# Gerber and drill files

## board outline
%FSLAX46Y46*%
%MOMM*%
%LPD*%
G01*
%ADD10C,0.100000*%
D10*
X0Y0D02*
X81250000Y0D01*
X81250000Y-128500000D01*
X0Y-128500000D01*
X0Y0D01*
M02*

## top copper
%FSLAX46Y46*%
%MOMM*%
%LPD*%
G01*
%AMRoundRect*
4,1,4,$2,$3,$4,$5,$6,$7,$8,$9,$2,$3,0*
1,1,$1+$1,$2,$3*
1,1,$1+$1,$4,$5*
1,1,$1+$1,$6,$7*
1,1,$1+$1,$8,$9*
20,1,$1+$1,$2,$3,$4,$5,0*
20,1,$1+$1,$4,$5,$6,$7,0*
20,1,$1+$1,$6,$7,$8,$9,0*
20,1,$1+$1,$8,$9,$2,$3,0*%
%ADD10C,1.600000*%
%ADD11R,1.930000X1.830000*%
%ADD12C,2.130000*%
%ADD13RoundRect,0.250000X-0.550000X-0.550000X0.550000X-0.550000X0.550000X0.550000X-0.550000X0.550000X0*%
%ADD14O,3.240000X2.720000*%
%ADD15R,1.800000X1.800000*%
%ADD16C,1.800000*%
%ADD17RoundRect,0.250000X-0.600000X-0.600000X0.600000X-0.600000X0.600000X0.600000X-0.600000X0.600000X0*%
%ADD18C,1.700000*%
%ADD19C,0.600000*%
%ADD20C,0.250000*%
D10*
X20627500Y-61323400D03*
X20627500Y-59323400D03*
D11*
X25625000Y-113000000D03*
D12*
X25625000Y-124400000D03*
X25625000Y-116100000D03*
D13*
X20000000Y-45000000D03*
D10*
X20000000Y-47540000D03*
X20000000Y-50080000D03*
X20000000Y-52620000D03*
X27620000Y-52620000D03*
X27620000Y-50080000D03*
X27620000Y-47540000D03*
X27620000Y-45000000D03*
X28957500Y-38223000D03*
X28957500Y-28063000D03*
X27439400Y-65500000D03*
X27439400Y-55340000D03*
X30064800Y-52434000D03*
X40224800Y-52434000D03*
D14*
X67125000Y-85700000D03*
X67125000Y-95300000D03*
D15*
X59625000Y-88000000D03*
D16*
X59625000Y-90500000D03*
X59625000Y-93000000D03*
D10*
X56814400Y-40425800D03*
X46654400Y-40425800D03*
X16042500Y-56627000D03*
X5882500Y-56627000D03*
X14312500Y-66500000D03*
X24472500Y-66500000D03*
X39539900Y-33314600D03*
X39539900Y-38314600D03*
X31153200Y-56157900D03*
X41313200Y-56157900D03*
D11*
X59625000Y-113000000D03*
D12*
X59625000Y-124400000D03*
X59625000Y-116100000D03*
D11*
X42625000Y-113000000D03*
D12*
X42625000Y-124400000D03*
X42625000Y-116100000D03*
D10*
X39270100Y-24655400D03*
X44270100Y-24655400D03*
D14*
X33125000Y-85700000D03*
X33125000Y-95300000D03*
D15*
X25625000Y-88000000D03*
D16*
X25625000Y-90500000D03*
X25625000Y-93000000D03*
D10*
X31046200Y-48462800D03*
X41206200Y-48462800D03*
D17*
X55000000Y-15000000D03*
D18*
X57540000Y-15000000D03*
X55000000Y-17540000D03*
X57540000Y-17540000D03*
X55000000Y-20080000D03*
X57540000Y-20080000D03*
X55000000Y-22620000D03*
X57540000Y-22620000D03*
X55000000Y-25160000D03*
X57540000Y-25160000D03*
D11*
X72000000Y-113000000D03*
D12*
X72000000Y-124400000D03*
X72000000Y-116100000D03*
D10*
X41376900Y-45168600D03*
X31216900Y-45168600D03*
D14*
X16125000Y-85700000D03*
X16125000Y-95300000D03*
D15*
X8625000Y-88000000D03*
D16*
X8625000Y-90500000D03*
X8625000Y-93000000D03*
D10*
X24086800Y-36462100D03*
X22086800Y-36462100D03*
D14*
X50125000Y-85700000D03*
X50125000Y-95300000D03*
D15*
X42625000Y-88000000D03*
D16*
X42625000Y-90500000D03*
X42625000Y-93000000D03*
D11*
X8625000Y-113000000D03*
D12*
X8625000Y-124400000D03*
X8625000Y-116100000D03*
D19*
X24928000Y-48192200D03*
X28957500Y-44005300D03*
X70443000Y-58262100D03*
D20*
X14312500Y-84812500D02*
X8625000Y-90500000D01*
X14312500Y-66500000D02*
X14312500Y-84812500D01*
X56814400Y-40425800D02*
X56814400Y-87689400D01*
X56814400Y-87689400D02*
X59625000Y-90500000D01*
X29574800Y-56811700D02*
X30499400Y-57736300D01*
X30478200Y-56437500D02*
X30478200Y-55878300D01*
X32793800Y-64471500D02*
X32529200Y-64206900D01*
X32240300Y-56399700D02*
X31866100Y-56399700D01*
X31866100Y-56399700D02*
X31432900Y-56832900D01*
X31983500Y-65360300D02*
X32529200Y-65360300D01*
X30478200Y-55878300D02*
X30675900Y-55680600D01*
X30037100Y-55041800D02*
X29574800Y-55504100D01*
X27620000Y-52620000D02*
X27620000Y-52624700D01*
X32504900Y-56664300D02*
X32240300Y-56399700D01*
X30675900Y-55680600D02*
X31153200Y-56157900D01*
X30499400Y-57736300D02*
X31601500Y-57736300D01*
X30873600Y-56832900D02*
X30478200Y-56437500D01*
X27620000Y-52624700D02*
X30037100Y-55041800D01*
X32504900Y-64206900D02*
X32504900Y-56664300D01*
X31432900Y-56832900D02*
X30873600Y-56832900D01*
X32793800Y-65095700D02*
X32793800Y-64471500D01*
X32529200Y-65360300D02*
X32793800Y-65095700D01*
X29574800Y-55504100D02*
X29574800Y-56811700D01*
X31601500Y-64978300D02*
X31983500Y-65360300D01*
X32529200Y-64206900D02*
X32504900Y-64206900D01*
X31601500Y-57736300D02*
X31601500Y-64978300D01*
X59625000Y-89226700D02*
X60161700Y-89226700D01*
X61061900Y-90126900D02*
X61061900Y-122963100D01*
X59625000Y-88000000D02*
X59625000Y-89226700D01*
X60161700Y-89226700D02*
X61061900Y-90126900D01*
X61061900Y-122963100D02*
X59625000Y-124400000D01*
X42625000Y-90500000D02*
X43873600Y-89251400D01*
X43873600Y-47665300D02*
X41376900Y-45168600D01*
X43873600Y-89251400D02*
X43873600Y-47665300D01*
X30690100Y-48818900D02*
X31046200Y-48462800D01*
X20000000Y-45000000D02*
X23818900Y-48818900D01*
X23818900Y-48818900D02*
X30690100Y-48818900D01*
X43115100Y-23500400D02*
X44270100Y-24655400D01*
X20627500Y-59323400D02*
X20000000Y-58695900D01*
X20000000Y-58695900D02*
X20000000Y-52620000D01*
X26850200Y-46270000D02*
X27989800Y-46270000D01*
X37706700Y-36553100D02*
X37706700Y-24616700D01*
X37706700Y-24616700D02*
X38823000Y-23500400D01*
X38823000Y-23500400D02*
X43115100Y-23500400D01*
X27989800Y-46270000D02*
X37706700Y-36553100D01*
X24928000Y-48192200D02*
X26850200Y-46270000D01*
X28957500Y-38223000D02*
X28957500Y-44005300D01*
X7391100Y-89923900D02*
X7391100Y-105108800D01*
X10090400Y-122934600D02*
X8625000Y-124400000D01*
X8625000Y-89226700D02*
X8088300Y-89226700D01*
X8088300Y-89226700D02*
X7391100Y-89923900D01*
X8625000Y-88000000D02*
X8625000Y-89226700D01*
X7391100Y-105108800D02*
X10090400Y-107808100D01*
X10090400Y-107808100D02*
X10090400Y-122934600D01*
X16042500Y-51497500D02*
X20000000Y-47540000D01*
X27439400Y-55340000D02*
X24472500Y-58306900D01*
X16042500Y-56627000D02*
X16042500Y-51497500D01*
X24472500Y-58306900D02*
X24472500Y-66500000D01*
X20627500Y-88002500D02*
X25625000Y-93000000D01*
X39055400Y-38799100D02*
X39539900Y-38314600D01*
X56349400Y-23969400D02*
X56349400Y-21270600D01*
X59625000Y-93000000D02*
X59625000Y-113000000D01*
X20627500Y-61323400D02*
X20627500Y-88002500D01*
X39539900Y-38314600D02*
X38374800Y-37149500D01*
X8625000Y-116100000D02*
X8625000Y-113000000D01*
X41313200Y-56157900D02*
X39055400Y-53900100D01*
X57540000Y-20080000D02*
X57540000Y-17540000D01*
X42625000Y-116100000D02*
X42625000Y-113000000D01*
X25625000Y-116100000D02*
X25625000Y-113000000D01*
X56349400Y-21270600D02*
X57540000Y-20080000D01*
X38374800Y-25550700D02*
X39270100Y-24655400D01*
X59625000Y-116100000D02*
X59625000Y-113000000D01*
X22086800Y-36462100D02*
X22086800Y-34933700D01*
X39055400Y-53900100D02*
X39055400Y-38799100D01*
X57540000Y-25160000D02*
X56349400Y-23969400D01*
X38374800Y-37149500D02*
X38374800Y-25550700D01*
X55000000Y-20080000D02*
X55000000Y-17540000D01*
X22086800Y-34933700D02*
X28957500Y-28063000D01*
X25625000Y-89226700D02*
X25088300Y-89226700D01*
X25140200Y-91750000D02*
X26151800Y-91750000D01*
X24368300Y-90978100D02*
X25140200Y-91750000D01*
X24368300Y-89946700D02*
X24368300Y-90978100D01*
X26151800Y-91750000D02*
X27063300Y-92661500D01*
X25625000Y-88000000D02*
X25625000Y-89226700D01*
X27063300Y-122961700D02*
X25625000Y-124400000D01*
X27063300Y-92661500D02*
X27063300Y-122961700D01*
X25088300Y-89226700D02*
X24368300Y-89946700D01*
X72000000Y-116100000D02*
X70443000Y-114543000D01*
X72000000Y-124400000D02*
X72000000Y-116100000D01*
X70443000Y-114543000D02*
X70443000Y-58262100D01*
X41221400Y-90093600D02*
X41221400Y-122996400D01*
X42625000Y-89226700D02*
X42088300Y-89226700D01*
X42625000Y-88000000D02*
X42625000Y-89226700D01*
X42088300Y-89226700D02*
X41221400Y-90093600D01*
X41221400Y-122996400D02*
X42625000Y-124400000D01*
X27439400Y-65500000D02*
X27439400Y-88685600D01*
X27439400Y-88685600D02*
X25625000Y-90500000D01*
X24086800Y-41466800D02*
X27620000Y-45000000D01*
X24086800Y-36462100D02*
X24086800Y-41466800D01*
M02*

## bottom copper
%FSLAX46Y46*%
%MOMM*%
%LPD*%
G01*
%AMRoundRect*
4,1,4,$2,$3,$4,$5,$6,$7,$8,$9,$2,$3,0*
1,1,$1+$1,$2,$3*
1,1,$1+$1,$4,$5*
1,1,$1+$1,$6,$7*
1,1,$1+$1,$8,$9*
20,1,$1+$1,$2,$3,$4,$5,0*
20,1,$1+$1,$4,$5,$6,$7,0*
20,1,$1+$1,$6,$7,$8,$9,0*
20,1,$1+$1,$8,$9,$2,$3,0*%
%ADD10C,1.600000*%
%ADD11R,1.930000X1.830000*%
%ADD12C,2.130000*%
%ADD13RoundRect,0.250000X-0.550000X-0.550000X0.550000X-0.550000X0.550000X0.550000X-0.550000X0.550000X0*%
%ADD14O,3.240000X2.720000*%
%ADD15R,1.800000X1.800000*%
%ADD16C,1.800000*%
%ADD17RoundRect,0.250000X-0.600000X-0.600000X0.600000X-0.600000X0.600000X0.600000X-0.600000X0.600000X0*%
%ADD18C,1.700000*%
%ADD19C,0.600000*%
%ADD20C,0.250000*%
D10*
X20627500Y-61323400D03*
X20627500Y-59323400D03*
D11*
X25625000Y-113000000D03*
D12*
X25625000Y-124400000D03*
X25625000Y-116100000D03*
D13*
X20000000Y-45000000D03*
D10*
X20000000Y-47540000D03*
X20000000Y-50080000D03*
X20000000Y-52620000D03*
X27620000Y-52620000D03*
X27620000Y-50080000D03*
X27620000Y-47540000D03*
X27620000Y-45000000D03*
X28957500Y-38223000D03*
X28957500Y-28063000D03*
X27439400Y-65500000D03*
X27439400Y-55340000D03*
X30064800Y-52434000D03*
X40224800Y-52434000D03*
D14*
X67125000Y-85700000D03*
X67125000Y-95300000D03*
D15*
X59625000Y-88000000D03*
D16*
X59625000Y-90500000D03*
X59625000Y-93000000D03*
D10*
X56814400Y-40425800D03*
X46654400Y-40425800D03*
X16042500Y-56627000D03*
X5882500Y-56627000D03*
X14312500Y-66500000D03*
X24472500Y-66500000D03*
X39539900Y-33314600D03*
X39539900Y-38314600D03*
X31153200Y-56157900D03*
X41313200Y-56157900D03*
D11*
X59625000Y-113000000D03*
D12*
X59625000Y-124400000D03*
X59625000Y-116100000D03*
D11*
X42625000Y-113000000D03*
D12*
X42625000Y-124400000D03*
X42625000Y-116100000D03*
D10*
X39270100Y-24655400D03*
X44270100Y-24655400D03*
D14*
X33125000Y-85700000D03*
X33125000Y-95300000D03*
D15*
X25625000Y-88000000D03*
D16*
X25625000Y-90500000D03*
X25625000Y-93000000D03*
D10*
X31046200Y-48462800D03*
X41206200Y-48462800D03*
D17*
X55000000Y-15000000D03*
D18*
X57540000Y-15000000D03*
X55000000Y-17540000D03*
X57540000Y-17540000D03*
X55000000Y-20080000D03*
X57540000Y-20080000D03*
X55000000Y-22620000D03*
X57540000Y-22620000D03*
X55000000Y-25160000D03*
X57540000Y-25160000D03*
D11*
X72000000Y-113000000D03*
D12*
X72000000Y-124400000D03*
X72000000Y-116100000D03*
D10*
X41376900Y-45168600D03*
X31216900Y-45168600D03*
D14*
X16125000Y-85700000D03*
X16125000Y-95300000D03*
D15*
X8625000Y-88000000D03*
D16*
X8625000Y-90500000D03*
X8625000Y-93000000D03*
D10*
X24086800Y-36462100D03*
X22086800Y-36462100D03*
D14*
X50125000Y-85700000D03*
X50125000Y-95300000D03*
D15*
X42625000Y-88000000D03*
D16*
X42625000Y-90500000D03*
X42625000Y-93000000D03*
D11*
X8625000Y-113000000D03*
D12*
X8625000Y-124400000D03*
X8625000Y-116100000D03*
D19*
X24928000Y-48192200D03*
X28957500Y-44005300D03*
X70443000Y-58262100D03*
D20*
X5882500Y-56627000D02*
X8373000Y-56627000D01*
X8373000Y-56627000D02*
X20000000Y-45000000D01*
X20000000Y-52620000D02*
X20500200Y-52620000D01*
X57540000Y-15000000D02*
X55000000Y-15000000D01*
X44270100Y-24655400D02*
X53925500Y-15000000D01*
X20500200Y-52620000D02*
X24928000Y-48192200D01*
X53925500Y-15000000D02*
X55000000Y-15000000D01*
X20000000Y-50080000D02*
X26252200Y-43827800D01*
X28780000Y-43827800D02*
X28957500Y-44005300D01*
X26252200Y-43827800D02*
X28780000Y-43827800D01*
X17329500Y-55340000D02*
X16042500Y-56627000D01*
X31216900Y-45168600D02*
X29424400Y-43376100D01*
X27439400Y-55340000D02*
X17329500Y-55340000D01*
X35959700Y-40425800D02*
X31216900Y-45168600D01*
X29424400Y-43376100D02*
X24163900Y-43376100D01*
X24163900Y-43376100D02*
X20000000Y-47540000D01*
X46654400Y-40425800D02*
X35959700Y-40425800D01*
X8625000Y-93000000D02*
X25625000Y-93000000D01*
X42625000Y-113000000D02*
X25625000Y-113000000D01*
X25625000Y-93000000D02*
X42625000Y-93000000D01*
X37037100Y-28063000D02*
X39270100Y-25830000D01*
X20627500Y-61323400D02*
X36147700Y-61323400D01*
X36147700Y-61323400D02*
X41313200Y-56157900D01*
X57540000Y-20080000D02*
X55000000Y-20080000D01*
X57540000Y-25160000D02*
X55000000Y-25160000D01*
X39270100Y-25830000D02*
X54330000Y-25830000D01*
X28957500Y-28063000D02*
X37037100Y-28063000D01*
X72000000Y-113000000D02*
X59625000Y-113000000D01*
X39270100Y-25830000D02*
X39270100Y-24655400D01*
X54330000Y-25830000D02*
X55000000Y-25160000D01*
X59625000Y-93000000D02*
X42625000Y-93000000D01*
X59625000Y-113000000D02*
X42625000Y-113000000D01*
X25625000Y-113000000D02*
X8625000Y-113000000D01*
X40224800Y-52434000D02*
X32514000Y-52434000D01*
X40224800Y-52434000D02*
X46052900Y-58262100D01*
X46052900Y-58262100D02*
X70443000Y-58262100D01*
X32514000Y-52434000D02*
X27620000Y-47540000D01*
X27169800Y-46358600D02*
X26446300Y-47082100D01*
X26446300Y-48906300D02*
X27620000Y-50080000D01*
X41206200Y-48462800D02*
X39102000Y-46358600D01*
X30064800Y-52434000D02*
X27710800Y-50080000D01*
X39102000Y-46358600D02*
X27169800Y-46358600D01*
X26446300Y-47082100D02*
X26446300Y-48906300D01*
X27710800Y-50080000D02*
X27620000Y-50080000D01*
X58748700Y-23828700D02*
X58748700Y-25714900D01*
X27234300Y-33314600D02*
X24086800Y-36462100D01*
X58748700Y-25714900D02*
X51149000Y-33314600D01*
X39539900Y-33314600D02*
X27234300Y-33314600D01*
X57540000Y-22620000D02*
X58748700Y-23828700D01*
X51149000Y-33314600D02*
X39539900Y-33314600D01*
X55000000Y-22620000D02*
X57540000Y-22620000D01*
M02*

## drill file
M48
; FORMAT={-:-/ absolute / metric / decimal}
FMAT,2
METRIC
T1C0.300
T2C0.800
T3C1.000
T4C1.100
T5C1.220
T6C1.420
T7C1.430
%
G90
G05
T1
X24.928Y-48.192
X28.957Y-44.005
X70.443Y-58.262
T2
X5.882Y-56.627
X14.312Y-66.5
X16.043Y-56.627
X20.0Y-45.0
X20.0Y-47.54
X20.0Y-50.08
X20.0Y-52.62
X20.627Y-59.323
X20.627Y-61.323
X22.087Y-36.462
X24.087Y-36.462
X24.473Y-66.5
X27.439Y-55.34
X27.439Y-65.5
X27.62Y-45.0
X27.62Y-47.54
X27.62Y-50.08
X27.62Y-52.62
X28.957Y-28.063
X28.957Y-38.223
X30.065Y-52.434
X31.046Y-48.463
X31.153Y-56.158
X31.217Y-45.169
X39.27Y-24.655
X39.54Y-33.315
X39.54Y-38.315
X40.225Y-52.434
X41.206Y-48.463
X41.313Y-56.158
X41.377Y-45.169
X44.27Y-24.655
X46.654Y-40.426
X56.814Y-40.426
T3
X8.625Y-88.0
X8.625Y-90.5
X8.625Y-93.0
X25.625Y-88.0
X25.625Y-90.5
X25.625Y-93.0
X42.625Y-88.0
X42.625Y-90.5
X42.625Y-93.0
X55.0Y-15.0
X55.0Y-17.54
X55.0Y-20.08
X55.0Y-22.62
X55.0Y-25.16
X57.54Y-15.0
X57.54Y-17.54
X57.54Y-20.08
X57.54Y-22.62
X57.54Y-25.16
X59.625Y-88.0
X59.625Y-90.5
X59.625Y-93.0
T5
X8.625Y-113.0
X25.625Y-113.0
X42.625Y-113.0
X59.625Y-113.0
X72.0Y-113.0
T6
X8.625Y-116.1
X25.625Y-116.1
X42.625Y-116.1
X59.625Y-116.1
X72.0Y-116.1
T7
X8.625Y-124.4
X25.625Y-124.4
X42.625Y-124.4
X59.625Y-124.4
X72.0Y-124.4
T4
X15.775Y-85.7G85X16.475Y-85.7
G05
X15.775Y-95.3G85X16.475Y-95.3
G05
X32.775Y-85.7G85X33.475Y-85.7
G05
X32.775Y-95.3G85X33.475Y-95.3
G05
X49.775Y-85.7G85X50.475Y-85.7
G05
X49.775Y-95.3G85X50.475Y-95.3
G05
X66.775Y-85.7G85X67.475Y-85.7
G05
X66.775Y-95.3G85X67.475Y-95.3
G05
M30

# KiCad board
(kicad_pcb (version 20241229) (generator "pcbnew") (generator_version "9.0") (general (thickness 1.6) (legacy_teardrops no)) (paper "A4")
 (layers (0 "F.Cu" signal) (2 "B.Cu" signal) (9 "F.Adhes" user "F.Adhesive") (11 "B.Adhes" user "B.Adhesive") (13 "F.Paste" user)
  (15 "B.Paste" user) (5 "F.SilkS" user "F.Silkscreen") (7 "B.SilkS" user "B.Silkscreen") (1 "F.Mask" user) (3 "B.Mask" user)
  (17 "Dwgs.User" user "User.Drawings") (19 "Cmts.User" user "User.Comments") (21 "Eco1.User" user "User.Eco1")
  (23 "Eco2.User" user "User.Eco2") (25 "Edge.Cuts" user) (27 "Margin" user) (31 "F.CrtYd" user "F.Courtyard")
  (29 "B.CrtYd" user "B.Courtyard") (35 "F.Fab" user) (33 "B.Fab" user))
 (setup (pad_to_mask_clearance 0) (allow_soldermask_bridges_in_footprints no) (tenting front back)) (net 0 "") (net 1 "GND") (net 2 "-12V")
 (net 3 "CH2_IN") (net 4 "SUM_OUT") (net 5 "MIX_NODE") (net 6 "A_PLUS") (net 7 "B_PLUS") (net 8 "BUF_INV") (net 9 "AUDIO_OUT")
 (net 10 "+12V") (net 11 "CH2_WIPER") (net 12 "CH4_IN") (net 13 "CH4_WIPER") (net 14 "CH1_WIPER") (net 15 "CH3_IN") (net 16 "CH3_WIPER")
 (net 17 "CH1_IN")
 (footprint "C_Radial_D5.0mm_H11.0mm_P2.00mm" (layer "F.Cu") (at 20.6275 61.3234 90)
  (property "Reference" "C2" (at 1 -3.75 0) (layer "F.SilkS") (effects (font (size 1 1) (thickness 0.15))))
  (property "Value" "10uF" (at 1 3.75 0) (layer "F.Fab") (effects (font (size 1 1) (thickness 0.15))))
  (pad "1" thru_hole circle (at 0 0 90) (size 1.6 1.6) (drill 0.8) (layers "*.Cu" "*.Mask") (remove_unused_layers no) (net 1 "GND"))
  (pad "2" thru_hole circle (at 2 0 90) (size 1.6 1.6) (drill 0.8) (layers "*.Cu" "*.Mask") (remove_unused_layers no) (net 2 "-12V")))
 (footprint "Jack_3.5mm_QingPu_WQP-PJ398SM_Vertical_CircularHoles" (layer "F.Cu") (at 25.625 113)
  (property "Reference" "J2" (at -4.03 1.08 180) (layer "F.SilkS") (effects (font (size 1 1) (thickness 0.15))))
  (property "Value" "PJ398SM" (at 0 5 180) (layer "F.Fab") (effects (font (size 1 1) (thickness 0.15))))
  (pad "S" thru_hole rect (at 0 0 180) (size 1.93 1.83) (drill 1.22) (layers "*.Cu" "*.Mask") (remove_unused_layers no) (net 1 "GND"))
  (pad "T" thru_hole circle (at 0 11.4 180) (size 2.13 2.13) (drill 1.43) (layers "*.Cu" "*.Mask") (remove_unused_layers no)
   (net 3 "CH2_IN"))
  (pad "TN" thru_hole circle (at 0 3.1 180) (size 2.13 2.13) (drill 1.42) (layers "*.Cu" "*.Mask") (remove_unused_layers no) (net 1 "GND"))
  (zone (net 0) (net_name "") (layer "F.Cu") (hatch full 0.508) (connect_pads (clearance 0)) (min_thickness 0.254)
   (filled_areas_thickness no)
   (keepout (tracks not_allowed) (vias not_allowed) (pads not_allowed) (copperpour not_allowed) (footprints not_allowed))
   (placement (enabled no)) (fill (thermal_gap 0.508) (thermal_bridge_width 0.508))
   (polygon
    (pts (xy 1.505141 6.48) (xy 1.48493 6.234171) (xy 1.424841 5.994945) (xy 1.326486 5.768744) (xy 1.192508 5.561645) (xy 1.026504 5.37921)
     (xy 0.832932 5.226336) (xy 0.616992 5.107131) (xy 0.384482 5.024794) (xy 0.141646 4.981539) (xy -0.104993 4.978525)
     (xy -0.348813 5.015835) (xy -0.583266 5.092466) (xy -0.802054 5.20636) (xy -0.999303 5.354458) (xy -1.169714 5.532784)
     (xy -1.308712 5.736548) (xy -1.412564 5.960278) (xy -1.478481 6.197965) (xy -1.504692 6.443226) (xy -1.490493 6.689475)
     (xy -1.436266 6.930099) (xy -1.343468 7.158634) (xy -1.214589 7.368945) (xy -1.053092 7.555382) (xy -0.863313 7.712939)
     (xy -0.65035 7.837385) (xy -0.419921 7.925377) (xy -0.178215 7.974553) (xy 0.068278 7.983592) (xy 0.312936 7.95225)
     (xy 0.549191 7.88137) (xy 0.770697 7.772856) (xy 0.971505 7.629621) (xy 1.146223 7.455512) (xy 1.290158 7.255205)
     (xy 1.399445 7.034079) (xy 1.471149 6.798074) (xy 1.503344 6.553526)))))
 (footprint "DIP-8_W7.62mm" (layer "F.Cu") (at 20 45)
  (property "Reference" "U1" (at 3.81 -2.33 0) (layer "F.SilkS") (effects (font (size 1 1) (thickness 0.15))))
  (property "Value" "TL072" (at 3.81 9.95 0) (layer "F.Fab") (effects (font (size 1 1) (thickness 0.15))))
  (pad "1" thru_hole roundrect (at 0 0) (size 1.6 1.6) (drill 0.8) (layers "*.Cu" "*.Mask") (remove_unused_layers no)
   (roundrect_rratio 0.15625) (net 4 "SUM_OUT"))
  (pad "2" thru_hole circle (at 0 2.54) (size 1.6 1.6) (drill 0.8) (layers "*.Cu" "*.Mask") (remove_unused_layers no) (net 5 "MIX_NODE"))
  (pad "3" thru_hole circle (at 0 5.08) (size 1.6 1.6) (drill 0.8) (layers "*.Cu" "*.Mask") (remove_unused_layers no) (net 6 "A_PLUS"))
  (pad "4" thru_hole circle (at 0 7.62) (size 1.6 1.6) (drill 0.8) (layers "*.Cu" "*.Mask") (remove_unused_layers no) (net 2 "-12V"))
  (pad "5" thru_hole circle (at 7.62 7.62) (size 1.6 1.6) (drill 0.8) (layers "*.Cu" "*.Mask") (remove_unused_layers no) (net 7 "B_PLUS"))
  (pad "6" thru_hole circle (at 7.62 5.08) (size 1.6 1.6) (drill 0.8) (layers "*.Cu" "*.Mask") (remove_unused_layers no) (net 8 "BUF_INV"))
  (pad "7" thru_hole circle (at 7.62 2.54) (size 1.6 1.6) (drill 0.8) (layers "*.Cu" "*.Mask") (remove_unused_layers no) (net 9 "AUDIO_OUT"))
  (pad "8" thru_hole circle (at 7.62 0) (size 1.6 1.6) (drill 0.8) (layers "*.Cu" "*.Mask") (remove_unused_layers no) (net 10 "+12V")))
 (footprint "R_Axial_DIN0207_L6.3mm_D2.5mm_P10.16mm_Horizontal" (layer "F.Cu") (at 28.9575 38.223 90)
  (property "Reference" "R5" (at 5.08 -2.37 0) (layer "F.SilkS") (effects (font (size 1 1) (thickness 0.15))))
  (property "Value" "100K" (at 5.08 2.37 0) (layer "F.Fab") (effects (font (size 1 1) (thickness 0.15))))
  (pad "1" thru_hole circle (at 0 0 90) (size 1.6 1.6) (drill 0.8) (layers "*.Cu" "*.Mask") (remove_unused_layers no) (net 6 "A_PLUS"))
  (pad "2" thru_hole circle (at 10.16 0 90) (size 1.6 1.6) (drill 0.8) (layers "*.Cu" "*.Mask") (remove_unused_layers no) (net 1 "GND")))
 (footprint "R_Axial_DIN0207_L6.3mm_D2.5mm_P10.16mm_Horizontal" (layer "F.Cu") (at 27.4394 65.5 90)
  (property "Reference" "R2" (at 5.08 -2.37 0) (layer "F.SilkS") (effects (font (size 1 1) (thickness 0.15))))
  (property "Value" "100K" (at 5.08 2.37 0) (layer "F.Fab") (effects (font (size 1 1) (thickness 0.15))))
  (pad "1" thru_hole circle (at 0 0 90) (size 1.6 1.6) (drill 0.8) (layers "*.Cu" "*.Mask") (remove_unused_layers no) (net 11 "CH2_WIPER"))
  (pad "2" thru_hole circle (at 10.16 0 90) (size 1.6 1.6) (drill 0.8) (layers "*.Cu" "*.Mask") (remove_unused_layers no) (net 5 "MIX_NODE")))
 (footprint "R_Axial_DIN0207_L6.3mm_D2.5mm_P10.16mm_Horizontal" (layer "F.Cu") (at 30.0648 52.434)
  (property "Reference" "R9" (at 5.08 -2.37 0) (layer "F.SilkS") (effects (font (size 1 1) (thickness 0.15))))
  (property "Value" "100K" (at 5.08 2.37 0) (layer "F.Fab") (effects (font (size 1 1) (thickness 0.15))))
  (pad "1" thru_hole circle (at 0 0) (size 1.6 1.6) (drill 0.8) (layers "*.Cu" "*.Mask") (remove_unused_layers no) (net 8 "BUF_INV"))
  (pad "2" thru_hole circle (at 10.16 0) (size 1.6 1.6) (drill 0.8) (layers "*.Cu" "*.Mask") (remove_unused_layers no) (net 9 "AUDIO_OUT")))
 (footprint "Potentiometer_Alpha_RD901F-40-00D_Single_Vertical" (layer "F.Cu") (at 59.625 88)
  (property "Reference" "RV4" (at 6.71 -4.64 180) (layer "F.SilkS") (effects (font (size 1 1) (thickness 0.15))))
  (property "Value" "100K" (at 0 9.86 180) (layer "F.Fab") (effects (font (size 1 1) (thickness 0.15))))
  (pad "" thru_hole oval (at 7.5 -2.3 90) (size 2.72 3.24) (drill oval 1.1 1.8) (layers "*.Cu" "*.Mask") (remove_unused_layers no))
  (pad "" thru_hole oval (at 7.5 7.3 90) (size 2.72 3.24) (drill oval 1.1 1.8) (layers "*.Cu" "*.Mask") (remove_unused_layers no))
  (pad "1" thru_hole rect (at 0 0 90) (size 1.8 1.8) (drill 1) (layers "*.Cu" "*.Mask") (remove_unused_layers no) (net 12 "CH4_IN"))
  (pad "2" thru_hole circle (at 0 2.5 90) (size 1.8 1.8) (drill 1) (layers "*.Cu" "*.Mask") (remove_unused_layers no) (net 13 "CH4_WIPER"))
  (pad "3" thru_hole circle (at 0 5 90) (size 1.8 1.8) (drill 1) (layers "*.Cu" "*.Mask") (remove_unused_layers no) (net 1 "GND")))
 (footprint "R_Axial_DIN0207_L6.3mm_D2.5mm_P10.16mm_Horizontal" (layer "F.Cu") (at 56.8144 40.4258 180)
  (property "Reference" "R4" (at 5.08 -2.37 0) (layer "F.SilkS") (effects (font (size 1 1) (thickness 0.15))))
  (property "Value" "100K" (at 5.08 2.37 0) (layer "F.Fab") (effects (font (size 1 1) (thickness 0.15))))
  (pad "1" thru_hole circle (at 0 0 180) (size 1.6 1.6) (drill 0.8) (layers "*.Cu" "*.Mask") (remove_unused_layers no) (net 13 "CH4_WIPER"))
  (pad "2" thru_hole circle (at 10.16 0 180) (size 1.6 1.6) (drill 0.8) (layers "*.Cu" "*.Mask") (remove_unused_layers no)
   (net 5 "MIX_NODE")))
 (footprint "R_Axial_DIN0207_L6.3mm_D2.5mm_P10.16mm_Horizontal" (layer "F.Cu") (at 16.0425 56.627 180)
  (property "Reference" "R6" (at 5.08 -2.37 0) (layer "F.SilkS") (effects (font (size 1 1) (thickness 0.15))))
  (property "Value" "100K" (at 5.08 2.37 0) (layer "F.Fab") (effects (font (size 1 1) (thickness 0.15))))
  (pad "1" thru_hole circle (at 0 0 180) (size 1.6 1.6) (drill 0.8) (layers "*.Cu" "*.Mask") (remove_unused_layers no) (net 5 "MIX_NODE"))
  (pad "2" thru_hole circle (at 10.16 0 180) (size 1.6 1.6) (drill 0.8) (layers "*.Cu" "*.Mask") (remove_unused_layers no) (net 4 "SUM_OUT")))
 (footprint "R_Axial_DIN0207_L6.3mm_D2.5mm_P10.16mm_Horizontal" (layer "F.Cu") (at 14.3125 66.5)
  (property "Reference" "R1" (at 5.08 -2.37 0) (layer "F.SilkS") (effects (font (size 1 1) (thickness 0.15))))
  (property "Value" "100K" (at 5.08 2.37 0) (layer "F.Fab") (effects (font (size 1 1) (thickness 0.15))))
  (pad "1" thru_hole circle (at 0 0) (size 1.6 1.6) (drill 0.8) (layers "*.Cu" "*.Mask") (remove_unused_layers no) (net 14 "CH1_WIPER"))
  (pad "2" thru_hole circle (at 10.16 0) (size 1.6 1.6) (drill 0.8) (layers "*.Cu" "*.Mask") (remove_unused_layers no) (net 5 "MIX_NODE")))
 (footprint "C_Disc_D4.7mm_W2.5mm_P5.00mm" (layer "F.Cu") (at 39.5399 33.3146 -90)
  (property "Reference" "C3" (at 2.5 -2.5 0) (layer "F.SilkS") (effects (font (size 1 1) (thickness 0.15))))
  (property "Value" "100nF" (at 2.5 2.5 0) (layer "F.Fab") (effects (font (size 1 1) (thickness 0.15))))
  (pad "1" thru_hole circle (at 0 0 270) (size 1.6 1.6) (drill 0.8) (layers "*.Cu" "*.Mask") (remove_unused_layers no) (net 10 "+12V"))
  (pad "2" thru_hole circle (at 5 0 270) (size 1.6 1.6) (drill 0.8) (layers "*.Cu" "*.Mask") (remove_unused_layers no) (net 1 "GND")))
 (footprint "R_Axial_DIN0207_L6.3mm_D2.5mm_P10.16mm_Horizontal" (layer "F.Cu") (at 31.1532 56.1579)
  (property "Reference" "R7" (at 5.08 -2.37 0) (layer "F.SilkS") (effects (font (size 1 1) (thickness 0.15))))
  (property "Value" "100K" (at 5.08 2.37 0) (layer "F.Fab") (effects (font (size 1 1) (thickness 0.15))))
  (pad "1" thru_hole circle (at 0 0) (size 1.6 1.6) (drill 0.8) (layers "*.Cu" "*.Mask") (remove_unused_layers no) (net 7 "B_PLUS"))
  (pad "2" thru_hole circle (at 10.16 0) (size 1.6 1.6) (drill 0.8) (layers "*.Cu" "*.Mask") (remove_unused_layers no) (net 1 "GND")))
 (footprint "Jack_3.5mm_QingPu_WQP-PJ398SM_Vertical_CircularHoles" (layer "F.Cu") (at 59.625 113)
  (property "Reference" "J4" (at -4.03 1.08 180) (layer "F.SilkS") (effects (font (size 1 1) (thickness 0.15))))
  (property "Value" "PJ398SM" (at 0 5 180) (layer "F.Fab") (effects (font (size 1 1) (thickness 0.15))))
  (pad "S" thru_hole rect (at 0 0 180) (size 1.93 1.83) (drill 1.22) (layers "*.Cu" "*.Mask") (remove_unused_layers no) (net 1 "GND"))
  (pad "T" thru_hole circle (at 0 11.4 180) (size 2.13 2.13) (drill 1.43) (layers "*.Cu" "*.Mask") (remove_unused_layers no)
   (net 12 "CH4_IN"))
  (pad "TN" thru_hole circle (at 0 3.1 180) (size 2.13 2.13) (drill 1.42) (layers "*.Cu" "*.Mask") (remove_unused_layers no) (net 1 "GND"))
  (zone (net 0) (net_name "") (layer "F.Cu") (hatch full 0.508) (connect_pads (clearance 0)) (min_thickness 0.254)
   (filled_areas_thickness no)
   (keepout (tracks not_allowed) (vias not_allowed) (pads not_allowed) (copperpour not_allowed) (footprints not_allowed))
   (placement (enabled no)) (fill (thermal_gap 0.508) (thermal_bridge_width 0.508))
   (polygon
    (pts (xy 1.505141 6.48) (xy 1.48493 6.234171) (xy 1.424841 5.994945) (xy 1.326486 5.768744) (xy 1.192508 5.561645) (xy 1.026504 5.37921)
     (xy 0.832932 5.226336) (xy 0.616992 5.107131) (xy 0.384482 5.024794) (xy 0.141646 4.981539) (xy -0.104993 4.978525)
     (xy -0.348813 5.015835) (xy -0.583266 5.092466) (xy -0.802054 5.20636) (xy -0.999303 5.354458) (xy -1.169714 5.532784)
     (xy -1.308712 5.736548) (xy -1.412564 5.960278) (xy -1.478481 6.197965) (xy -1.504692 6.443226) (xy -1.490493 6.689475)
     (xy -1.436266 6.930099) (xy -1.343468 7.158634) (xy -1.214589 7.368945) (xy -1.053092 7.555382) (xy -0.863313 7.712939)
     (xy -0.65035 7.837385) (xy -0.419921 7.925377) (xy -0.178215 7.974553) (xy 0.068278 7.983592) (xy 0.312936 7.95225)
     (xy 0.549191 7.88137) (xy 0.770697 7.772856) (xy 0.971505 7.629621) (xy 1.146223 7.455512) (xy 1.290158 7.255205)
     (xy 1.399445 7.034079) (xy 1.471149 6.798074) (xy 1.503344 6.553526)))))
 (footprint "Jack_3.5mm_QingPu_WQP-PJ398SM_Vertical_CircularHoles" (layer "F.Cu") (at 42.625 113)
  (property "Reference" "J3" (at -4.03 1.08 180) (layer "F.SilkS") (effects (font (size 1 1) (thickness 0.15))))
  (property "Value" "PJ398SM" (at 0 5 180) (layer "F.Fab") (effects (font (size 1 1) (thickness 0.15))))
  (pad "S" thru_hole rect (at 0 0 180) (size 1.93 1.83) (drill 1.22) (layers "*.Cu" "*.Mask") (remove_unused_layers no) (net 1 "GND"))
  (pad "T" thru_hole circle (at 0 11.4 180) (size 2.13 2.13) (drill 1.43) (layers "*.Cu" "*.Mask") (remove_unused_layers no)
   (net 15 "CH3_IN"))
  (pad "TN" thru_hole circle (at 0 3.1 180) (size 2.13 2.13) (drill 1.42) (layers "*.Cu" "*.Mask") (remove_unused_layers no) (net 1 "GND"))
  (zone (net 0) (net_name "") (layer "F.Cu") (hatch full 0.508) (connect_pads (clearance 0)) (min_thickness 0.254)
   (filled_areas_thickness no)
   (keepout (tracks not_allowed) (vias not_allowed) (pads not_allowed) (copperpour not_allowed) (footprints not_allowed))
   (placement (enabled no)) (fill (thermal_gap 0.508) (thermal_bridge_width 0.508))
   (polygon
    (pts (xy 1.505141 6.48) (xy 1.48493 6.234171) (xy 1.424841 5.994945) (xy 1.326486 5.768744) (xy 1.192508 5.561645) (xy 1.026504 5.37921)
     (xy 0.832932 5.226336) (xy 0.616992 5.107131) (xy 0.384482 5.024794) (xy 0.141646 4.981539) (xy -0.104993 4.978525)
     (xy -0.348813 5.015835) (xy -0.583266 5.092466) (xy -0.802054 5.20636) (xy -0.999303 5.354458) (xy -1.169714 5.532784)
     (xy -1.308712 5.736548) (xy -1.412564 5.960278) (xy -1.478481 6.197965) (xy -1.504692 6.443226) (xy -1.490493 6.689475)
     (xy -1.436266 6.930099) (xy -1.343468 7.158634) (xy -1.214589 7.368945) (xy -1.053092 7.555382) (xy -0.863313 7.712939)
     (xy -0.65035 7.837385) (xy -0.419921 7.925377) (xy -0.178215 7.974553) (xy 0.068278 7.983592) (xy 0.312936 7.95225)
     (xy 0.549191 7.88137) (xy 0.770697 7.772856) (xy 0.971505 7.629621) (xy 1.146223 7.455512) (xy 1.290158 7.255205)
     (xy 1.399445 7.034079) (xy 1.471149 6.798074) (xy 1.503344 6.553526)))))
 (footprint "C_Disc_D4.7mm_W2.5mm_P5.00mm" (layer "F.Cu") (at 39.2701 24.6554)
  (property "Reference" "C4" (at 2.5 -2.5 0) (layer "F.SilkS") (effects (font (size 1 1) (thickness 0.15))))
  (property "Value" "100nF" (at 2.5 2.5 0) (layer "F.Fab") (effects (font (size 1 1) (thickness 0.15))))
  (pad "1" thru_hole circle (at 0 0) (size 1.6 1.6) (drill 0.8) (layers "*.Cu" "*.Mask") (remove_unused_layers no) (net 1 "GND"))
  (pad "2" thru_hole circle (at 5 0) (size 1.6 1.6) (drill 0.8) (layers "*.Cu" "*.Mask") (remove_unused_layers no) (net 2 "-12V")))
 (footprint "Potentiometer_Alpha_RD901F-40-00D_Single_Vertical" (layer "F.Cu") (at 25.625 88)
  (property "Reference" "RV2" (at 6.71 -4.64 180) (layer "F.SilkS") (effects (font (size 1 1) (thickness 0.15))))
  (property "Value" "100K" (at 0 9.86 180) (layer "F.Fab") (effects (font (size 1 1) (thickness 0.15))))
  (pad "" thru_hole oval (at 7.5 -2.3 90) (size 2.72 3.24) (drill oval 1.1 1.8) (layers "*.Cu" "*.Mask") (remove_unused_layers no))
  (pad "" thru_hole oval (at 7.5 7.3 90) (size 2.72 3.24) (drill oval 1.1 1.8) (layers "*.Cu" "*.Mask") (remove_unused_layers no))
  (pad "1" thru_hole rect (at 0 0 90) (size 1.8 1.8) (drill 1) (layers "*.Cu" "*.Mask") (remove_unused_layers no) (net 3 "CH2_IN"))
  (pad "2" thru_hole circle (at 0 2.5 90) (size 1.8 1.8) (drill 1) (layers "*.Cu" "*.Mask") (remove_unused_layers no) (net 11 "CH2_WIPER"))
  (pad "3" thru_hole circle (at 0 5 90) (size 1.8 1.8) (drill 1) (layers "*.Cu" "*.Mask") (remove_unused_layers no) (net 1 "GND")))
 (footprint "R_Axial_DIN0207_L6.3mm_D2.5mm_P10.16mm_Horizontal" (layer "F.Cu") (at 31.0462 48.4628)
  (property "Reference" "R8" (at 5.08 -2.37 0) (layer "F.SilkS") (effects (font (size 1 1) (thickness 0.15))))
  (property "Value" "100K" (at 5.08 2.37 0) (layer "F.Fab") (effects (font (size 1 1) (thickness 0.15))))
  (pad "1" thru_hole circle (at 0 0) (size 1.6 1.6) (drill 0.8) (layers "*.Cu" "*.Mask") (remove_unused_layers no) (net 4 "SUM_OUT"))
  (pad "2" thru_hole circle (at 10.16 0) (size 1.6 1.6) (drill 0.8) (layers "*.Cu" "*.Mask") (remove_unused_layers no) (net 8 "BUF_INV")))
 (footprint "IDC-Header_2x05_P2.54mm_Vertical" (layer "F.Cu") (at 55 15)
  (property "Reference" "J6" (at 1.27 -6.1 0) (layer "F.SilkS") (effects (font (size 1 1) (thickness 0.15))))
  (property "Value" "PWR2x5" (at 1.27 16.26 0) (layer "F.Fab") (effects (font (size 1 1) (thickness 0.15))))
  (pad "1" thru_hole roundrect (at 0 0) (size 1.7 1.7) (drill 1) (layers "*.Cu" "*.Mask") (remove_unused_layers no)
   (roundrect_rratio 0.147059) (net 2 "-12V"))
  (pad "2" thru_hole circle (at 2.54 0) (size 1.7 1.7) (drill 1) (layers "*.Cu" "*.Mask") (remove_unused_layers no) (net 2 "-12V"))
  (pad "3" thru_hole circle (at 0 2.54) (size 1.7 1.7) (drill 1) (layers "*.Cu" "*.Mask") (remove_unused_layers no) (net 1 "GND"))
  (pad "4" thru_hole circle (at 2.54 2.54) (size 1.7 1.7) (drill 1) (layers "*.Cu" "*.Mask") (remove_unused_layers no) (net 1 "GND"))
  (pad "5" thru_hole circle (at 0 5.08) (size 1.7 1.7) (drill 1) (layers "*.Cu" "*.Mask") (remove_unused_layers no) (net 1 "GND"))
  (pad "6" thru_hole circle (at 2.54 5.08) (size 1.7 1.7) (drill 1) (layers "*.Cu" "*.Mask") (remove_unused_layers no) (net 1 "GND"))
  (pad "7" thru_hole circle (at 0 7.62) (size 1.7 1.7) (drill 1) (layers "*.Cu" "*.Mask") (remove_unused_layers no) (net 10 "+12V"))
  (pad "8" thru_hole circle (at 2.54 7.62) (size 1.7 1.7) (drill 1) (layers "*.Cu" "*.Mask") (remove_unused_layers no) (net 10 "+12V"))
  (pad "9" thru_hole circle (at 0 10.16) (size 1.7 1.7) (drill 1) (layers "*.Cu" "*.Mask") (remove_unused_layers no) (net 1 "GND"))
  (pad "10" thru_hole circle (at 2.54 10.16) (size 1.7 1.7) (drill 1) (layers "*.Cu" "*.Mask") (remove_unused_layers no) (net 1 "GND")))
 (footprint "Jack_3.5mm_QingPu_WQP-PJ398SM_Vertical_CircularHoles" (layer "F.Cu") (at 72 113)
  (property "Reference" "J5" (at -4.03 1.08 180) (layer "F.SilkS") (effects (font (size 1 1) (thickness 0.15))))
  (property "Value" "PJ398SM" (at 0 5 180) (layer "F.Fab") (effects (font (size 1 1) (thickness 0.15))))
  (pad "S" thru_hole rect (at 0 0 180) (size 1.93 1.83) (drill 1.22) (layers "*.Cu" "*.Mask") (remove_unused_layers no) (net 1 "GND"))
  (pad "T" thru_hole circle (at 0 11.4 180) (size 2.13 2.13) (drill 1.43) (layers "*.Cu" "*.Mask") (remove_unused_layers no)
   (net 9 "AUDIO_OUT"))
  (pad "TN" thru_hole circle (at 0 3.1 180) (size 2.13 2.13) (drill 1.42) (layers "*.Cu" "*.Mask") (remove_unused_layers no)
   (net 9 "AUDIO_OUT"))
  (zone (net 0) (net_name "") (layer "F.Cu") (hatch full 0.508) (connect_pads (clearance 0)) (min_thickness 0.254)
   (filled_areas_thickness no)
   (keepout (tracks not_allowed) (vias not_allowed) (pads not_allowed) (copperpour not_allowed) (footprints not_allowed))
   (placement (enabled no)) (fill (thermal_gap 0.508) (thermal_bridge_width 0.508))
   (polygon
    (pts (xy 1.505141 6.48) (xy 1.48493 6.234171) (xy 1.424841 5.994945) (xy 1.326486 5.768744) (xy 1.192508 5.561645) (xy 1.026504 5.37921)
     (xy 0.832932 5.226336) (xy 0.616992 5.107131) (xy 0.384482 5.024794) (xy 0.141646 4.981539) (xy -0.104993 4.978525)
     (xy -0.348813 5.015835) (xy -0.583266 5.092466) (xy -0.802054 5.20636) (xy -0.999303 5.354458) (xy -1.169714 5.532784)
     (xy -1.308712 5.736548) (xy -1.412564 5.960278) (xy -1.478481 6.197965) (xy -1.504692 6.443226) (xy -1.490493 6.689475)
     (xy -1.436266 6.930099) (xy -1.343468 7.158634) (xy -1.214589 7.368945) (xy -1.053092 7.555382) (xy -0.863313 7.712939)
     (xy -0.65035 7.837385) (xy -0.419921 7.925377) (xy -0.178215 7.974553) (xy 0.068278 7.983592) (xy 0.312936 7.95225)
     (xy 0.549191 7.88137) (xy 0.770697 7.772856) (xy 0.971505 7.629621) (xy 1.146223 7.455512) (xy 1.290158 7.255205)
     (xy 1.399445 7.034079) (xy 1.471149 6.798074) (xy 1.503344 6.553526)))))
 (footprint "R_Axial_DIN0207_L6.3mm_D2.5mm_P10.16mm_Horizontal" (layer "F.Cu") (at 41.3769 45.1686 180)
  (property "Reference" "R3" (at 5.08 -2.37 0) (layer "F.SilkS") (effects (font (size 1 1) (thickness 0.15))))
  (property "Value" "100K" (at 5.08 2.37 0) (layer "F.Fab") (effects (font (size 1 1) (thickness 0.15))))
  (pad "1" thru_hole circle (at 0 0 180) (size 1.6 1.6) (drill 0.8) (layers "*.Cu" "*.Mask") (remove_unused_layers no) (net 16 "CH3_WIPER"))
  (pad "2" thru_hole circle (at 10.16 0 180) (size 1.6 1.6) (drill 0.8) (layers "*.Cu" "*.Mask") (remove_unused_layers no)
   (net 5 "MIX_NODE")))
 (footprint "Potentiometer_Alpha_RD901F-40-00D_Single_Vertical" (layer "F.Cu") (at 8.625 88)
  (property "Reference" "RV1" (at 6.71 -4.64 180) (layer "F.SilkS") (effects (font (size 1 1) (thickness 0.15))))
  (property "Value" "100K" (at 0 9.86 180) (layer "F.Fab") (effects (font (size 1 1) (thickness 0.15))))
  (pad "" thru_hole oval (at 7.5 -2.3 90) (size 2.72 3.24) (drill oval 1.1 1.8) (layers "*.Cu" "*.Mask") (remove_unused_layers no))
  (pad "" thru_hole oval (at 7.5 7.3 90) (size 2.72 3.24) (drill oval 1.1 1.8) (layers "*.Cu" "*.Mask") (remove_unused_layers no))
  (pad "1" thru_hole rect (at 0 0 90) (size 1.8 1.8) (drill 1) (layers "*.Cu" "*.Mask") (remove_unused_layers no) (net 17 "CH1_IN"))
  (pad "2" thru_hole circle (at 0 2.5 90) (size 1.8 1.8) (drill 1) (layers "*.Cu" "*.Mask") (remove_unused_layers no) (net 14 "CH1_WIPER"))
  (pad "3" thru_hole circle (at 0 5 90) (size 1.8 1.8) (drill 1) (layers "*.Cu" "*.Mask") (remove_unused_layers no) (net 1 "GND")))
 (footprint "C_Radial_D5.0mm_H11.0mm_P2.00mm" (layer "F.Cu") (at 24.0868 36.4621 180)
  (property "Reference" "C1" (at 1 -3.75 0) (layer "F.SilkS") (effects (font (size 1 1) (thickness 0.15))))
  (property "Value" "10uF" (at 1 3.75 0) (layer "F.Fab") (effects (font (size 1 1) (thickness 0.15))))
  (pad "1" thru_hole circle (at 0 0 180) (size 1.6 1.6) (drill 0.8) (layers "*.Cu" "*.Mask") (remove_unused_layers no) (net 10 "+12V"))
  (pad "2" thru_hole circle (at 2 0 180) (size 1.6 1.6) (drill 0.8) (layers "*.Cu" "*.Mask") (remove_unused_layers no) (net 1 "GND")))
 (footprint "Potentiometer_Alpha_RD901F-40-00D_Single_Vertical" (layer "F.Cu") (at 42.625 88)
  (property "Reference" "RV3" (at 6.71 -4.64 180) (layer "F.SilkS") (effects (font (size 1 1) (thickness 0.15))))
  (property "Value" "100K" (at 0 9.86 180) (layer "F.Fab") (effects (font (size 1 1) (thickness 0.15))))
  (pad "" thru_hole oval (at 7.5 -2.3 90) (size 2.72 3.24) (drill oval 1.1 1.8) (layers "*.Cu" "*.Mask") (remove_unused_layers no))
  (pad "" thru_hole oval (at 7.5 7.3 90) (size 2.72 3.24) (drill oval 1.1 1.8) (layers "*.Cu" "*.Mask") (remove_unused_layers no))
  (pad "1" thru_hole rect (at 0 0 90) (size 1.8 1.8) (drill 1) (layers "*.Cu" "*.Mask") (remove_unused_layers no) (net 15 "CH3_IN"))
  (pad "2" thru_hole circle (at 0 2.5 90) (size 1.8 1.8) (drill 1) (layers "*.Cu" "*.Mask") (remove_unused_layers no) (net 16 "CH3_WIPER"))
  (pad "3" thru_hole circle (at 0 5 90) (size 1.8 1.8) (drill 1) (layers "*.Cu" "*.Mask") (remove_unused_layers no) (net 1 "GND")))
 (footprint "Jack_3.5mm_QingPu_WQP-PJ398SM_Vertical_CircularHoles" (layer "F.Cu") (at 8.625 113)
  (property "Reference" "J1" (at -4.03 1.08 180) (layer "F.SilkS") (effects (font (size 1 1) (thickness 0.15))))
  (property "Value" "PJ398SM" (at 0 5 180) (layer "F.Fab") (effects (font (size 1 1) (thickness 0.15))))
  (pad "S" thru_hole rect (at 0 0 180) (size 1.93 1.83) (drill 1.22) (layers "*.Cu" "*.Mask") (remove_unused_layers no) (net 1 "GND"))
  (pad "T" thru_hole circle (at 0 11.4 180) (size 2.13 2.13) (drill 1.43) (layers "*.Cu" "*.Mask") (remove_unused_layers no)
   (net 17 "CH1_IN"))
  (pad "TN" thru_hole circle (at 0 3.1 180) (size 2.13 2.13) (drill 1.42) (layers "*.Cu" "*.Mask") (remove_unused_layers no) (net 1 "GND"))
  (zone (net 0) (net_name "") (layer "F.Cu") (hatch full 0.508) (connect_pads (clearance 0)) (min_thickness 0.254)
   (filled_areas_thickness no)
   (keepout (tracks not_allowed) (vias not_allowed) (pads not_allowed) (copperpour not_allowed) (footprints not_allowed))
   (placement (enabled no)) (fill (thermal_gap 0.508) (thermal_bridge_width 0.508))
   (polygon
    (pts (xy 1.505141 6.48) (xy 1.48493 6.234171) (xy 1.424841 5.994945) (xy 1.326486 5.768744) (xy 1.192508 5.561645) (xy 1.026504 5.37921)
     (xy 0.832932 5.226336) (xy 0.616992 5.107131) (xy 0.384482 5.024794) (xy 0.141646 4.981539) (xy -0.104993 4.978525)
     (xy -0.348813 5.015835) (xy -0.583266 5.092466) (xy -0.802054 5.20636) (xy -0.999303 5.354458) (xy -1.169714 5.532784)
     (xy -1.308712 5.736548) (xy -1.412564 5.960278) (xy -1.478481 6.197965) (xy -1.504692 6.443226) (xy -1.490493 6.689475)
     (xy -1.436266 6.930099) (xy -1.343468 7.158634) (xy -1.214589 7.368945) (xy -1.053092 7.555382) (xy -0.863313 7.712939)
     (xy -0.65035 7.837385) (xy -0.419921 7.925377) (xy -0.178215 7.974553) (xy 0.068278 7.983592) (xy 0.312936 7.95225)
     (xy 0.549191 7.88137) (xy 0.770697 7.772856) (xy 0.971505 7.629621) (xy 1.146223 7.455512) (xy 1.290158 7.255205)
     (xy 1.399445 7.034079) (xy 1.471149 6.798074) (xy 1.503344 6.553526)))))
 (gr_rect (start 0 0) (end 81.25 128.5) (stroke (width 0.1) (type solid)) (fill no) (layer "Edge.Cuts"))
 (segment (start 14.3125 84.8125) (end 8.625 90.5) (width 0.25) (layer "F.Cu") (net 14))
 (segment (start 14.3125 66.5) (end 14.3125 84.8125) (width 0.25) (layer "F.Cu") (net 14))
 (segment (start 56.8144 40.4258) (end 56.8144 87.6894) (width 0.25) (layer "F.Cu") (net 13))
 (segment (start 56.8144 87.6894) (end 59.625 90.5) (width 0.25) (layer "F.Cu") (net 13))
 (segment (start 29.5748 56.8117) (end 30.4994 57.7363) (width 0.25) (layer "F.Cu") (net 7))
 (segment (start 30.4782 56.4375) (end 30.4782 55.8783) (width 0.25) (layer "F.Cu") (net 7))
 (segment (start 32.7938 64.4715) (end 32.5292 64.2069) (width 0.25) (layer "F.Cu") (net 7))
 (segment (start 32.2403 56.3997) (end 31.8661 56.3997) (width 0.25) (layer "F.Cu") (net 7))
 (segment (start 31.8661 56.3997) (end 31.4329 56.8329) (width 0.25) (layer "F.Cu") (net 7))
 (segment (start 31.9835 65.3603) (end 32.5292 65.3603) (width 0.25) (layer "F.Cu") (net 7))
 (segment (start 30.4782 55.8783) (end 30.6759 55.6806) (width 0.25) (layer "F.Cu") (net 7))
 (segment (start 30.0371 55.0418) (end 29.5748 55.5041) (width 0.25) (layer "F.Cu") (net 7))
 (segment (start 27.62 52.62) (end 27.62 52.6247) (width 0.25) (layer "F.Cu") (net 7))
 (segment (start 32.5049 56.6643) (end 32.2403 56.3997) (width 0.25) (layer "F.Cu") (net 7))
 (segment (start 30.6759 55.6806) (end 31.1532 56.1579) (width 0.25) (layer "F.Cu") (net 7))
 (segment (start 30.4994 57.7363) (end 31.6015 57.7363) (width 0.25) (layer "F.Cu") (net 7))
 (segment (start 30.8736 56.8329) (end 30.4782 56.4375) (width 0.25) (layer "F.Cu") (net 7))
 (segment (start 27.62 52.6247) (end 30.0371 55.0418) (width 0.25) (layer "F.Cu") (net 7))
 (segment (start 32.5049 64.2069) (end 32.5049 56.6643) (width 0.25) (layer "F.Cu") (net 7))
 (segment (start 31.4329 56.8329) (end 30.8736 56.8329) (width 0.25) (layer "F.Cu") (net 7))
 (segment (start 32.7938 65.0957) (end 32.7938 64.4715) (width 0.25) (layer "F.Cu") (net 7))
 (segment (start 32.5292 65.3603) (end 32.7938 65.0957) (width 0.25) (layer "F.Cu") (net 7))
 (segment (start 29.5748 55.5041) (end 29.5748 56.8117) (width 0.25) (layer "F.Cu") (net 7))
 (segment (start 31.6015 64.9783) (end 31.9835 65.3603) (width 0.25) (layer "F.Cu") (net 7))
 (segment (start 32.5292 64.2069) (end 32.5049 64.2069) (width 0.25) (layer "F.Cu") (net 7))
 (segment (start 31.6015 57.7363) (end 31.6015 64.9783) (width 0.25) (layer "F.Cu") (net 7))
 (segment (start 59.625 89.2267) (end 60.1617 89.2267) (width 0.25) (layer "F.Cu") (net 12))
 (segment (start 61.0619 90.1269) (end 61.0619 122.9631) (width 0.25) (layer "F.Cu") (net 12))
 (segment (start 59.625 88) (end 59.625 89.2267) (width 0.25) (layer "F.Cu") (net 12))
 (segment (start 60.1617 89.2267) (end 61.0619 90.1269) (width 0.25) (layer "F.Cu") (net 12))
 (segment (start 61.0619 122.9631) (end 59.625 124.4) (width 0.25) (layer "F.Cu") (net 12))
 (segment (start 42.625 90.5) (end 43.8736 89.2514) (width 0.25) (layer "F.Cu") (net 16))
 (segment (start 43.8736 47.6653) (end 41.3769 45.1686) (width 0.25) (layer "F.Cu") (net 16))
 (segment (start 43.8736 89.2514) (end 43.8736 47.6653) (width 0.25) (layer "F.Cu") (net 16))
 (segment (start 30.6901 48.8189) (end 31.0462 48.4628) (width 0.25) (layer "F.Cu") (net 4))
 (segment (start 20 45) (end 23.8189 48.8189) (width 0.25) (layer "F.Cu") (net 4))
 (segment (start 23.8189 48.8189) (end 30.6901 48.8189) (width 0.25) (layer "F.Cu") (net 4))
 (segment (start 5.8825 56.627) (end 8.373 56.627) (width 0.25) (layer "B.Cu") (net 4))
 (segment (start 8.373 56.627) (end 20 45) (width 0.25) (layer "B.Cu") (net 4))
 (segment (start 43.1151 23.5004) (end 44.2701 24.6554) (width 0.25) (layer "F.Cu") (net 2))
 (segment (start 20.6275 59.3234) (end 20 58.6959) (width 0.25) (layer "F.Cu") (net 2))
 (segment (start 20 58.6959) (end 20 52.62) (width 0.25) (layer "F.Cu") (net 2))
 (segment (start 26.8502 46.27) (end 27.9898 46.27) (width 0.25) (layer "F.Cu") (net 2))
 (segment (start 37.7067 36.5531) (end 37.7067 24.6167) (width 0.25) (layer "F.Cu") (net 2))
 (segment (start 37.7067 24.6167) (end 38.823 23.5004) (width 0.25) (layer "F.Cu") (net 2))
 (segment (start 38.823 23.5004) (end 43.1151 23.5004) (width 0.25) (layer "F.Cu") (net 2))
 (segment (start 27.9898 46.27) (end 37.7067 36.5531) (width 0.25) (layer "F.Cu") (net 2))
 (segment (start 24.928 48.1922) (end 26.8502 46.27) (width 0.25) (layer "F.Cu") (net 2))
 (via (at 24.928 48.1922) (size 0.6) (drill 0.3) (layers "F.Cu" "B.Cu") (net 2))
 (segment (start 20 52.62) (end 20.5002 52.62) (width 0.25) (layer "B.Cu") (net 2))
 (segment (start 57.54 15) (end 55 15) (width 0.25) (layer "B.Cu") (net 2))
 (segment (start 44.2701 24.6554) (end 53.9255 15) (width 0.25) (layer "B.Cu") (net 2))
 (segment (start 20.5002 52.62) (end 24.928 48.1922) (width 0.25) (layer "B.Cu") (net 2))
 (segment (start 53.9255 15) (end 55 15) (width 0.25) (layer "B.Cu") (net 2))
 (segment (start 28.9575 38.223) (end 28.9575 44.0053) (width 0.25) (layer "F.Cu") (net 6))
 (via (at 28.9575 44.0053) (size 0.6) (drill 0.3) (layers "F.Cu" "B.Cu") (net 6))
 (segment (start 20 50.08) (end 26.2522 43.8278) (width 0.25) (layer "B.Cu") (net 6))
 (segment (start 28.78 43.8278) (end 28.9575 44.0053) (width 0.25) (layer "B.Cu") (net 6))
 (segment (start 26.2522 43.8278) (end 28.78 43.8278) (width 0.25) (layer "B.Cu") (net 6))
 (segment (start 7.3911 89.9239) (end 7.3911 105.1088) (width 0.25) (layer "F.Cu") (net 17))
 (segment (start 10.0904 122.9346) (end 8.625 124.4) (width 0.25) (layer "F.Cu") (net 17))
 (segment (start 8.625 89.2267) (end 8.0883 89.2267) (width 0.25) (layer "F.Cu") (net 17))
 (segment (start 8.0883 89.2267) (end 7.3911 89.9239) (width 0.25) (layer "F.Cu") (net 17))
 (segment (start 8.625 88) (end 8.625 89.2267) (width 0.25) (layer "F.Cu") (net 17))
 (segment (start 7.3911 105.1088) (end 10.0904 107.8081) (width 0.25) (layer "F.Cu") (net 17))
 (segment (start 10.0904 107.8081) (end 10.0904 122.9346) (width 0.25) (layer "F.Cu") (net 17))
 (segment (start 16.0425 51.4975) (end 20 47.54) (width 0.25) (layer "F.Cu") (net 5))
 (segment (start 27.4394 55.34) (end 24.4725 58.3069) (width 0.25) (layer "F.Cu") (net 5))
 (segment (start 16.0425 56.627) (end 16.0425 51.4975) (width 0.25) (layer "F.Cu") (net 5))
 (segment (start 24.4725 58.3069) (end 24.4725 66.5) (width 0.25) (layer "F.Cu") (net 5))
 (segment (start 17.3295 55.34) (end 16.0425 56.627) (width 0.25) (layer "B.Cu") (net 5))
 (segment (start 31.2169 45.1686) (end 29.4244 43.3761) (width 0.25) (layer "B.Cu") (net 5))
 (segment (start 27.4394 55.34) (end 17.3295 55.34) (width 0.25) (layer "B.Cu") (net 5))
 (segment (start 35.9597 40.4258) (end 31.2169 45.1686) (width 0.25) (layer "B.Cu") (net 5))
 (segment (start 29.4244 43.3761) (end 24.1639 43.3761) (width 0.25) (layer "B.Cu") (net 5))
 (segment (start 24.1639 43.3761) (end 20 47.54) (width 0.25) (layer "B.Cu") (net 5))
 (segment (start 46.6544 40.4258) (end 35.9597 40.4258) (width 0.25) (layer "B.Cu") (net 5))
 (segment (start 20.6275 88.0025) (end 25.625 93) (width 0.25) (layer "F.Cu") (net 1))
 (segment (start 39.0554 38.7991) (end 39.5399 38.3146) (width 0.25) (layer "F.Cu") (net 1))
 (segment (start 56.3494 23.9694) (end 56.3494 21.2706) (width 0.25) (layer "F.Cu") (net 1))
 (segment (start 59.625 93) (end 59.625 113) (width 0.25) (layer "F.Cu") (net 1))
 (segment (start 20.6275 61.3234) (end 20.6275 88.0025) (width 0.25) (layer "F.Cu") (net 1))
 (segment (start 39.5399 38.3146) (end 38.3748 37.1495) (width 0.25) (layer "F.Cu") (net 1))
 (segment (start 8.625 116.1) (end 8.625 113) (width 0.25) (layer "F.Cu") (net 1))
 (segment (start 41.3132 56.1579) (end 39.0554 53.9001) (width 0.25) (layer "F.Cu") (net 1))
 (segment (start 57.54 20.08) (end 57.54 17.54) (width 0.25) (layer "F.Cu") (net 1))
 (segment (start 42.625 116.1) (end 42.625 113) (width 0.25) (layer "F.Cu") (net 1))
 (segment (start 25.625 116.1) (end 25.625 113) (width 0.25) (layer "F.Cu") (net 1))
 (segment (start 56.3494 21.2706) (end 57.54 20.08) (width 0.25) (layer "F.Cu") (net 1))
 (segment (start 38.3748 25.5507) (end 39.2701 24.6554) (width 0.25) (layer "F.Cu") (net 1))
 (segment (start 59.625 116.1) (end 59.625 113) (width 0.25) (layer "F.Cu") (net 1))
 (segment (start 22.0868 36.4621) (end 22.0868 34.9337) (width 0.25) (layer "F.Cu") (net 1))
 (segment (start 39.0554 53.9001) (end 39.0554 38.7991) (width 0.25) (layer "F.Cu") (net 1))
 (segment (start 57.54 25.16) (end 56.3494 23.9694) (width 0.25) (layer "F.Cu") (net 1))
 (segment (start 38.3748 37.1495) (end 38.3748 25.5507) (width 0.25) (layer "F.Cu") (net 1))
 (segment (start 55 20.08) (end 55 17.54) (width 0.25) (layer "F.Cu") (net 1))
 (segment (start 22.0868 34.9337) (end 28.9575 28.063) (width 0.25) (layer "F.Cu") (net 1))
 (segment (start 8.625 93) (end 25.625 93) (width 0.25) (layer "B.Cu") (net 1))
 (segment (start 42.625 113) (end 25.625 113) (width 0.25) (layer "B.Cu") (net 1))
 (segment (start 25.625 93) (end 42.625 93) (width 0.25) (layer "B.Cu") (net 1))
 (segment (start 37.0371 28.063) (end 39.2701 25.83) (width 0.25) (layer "B.Cu") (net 1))
 (segment (start 20.6275 61.3234) (end 36.1477 61.3234) (width 0.25) (layer "B.Cu") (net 1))
 (segment (start 36.1477 61.3234) (end 41.3132 56.1579) (width 0.25) (layer "B.Cu") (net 1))
 (segment (start 57.54 20.08) (end 55 20.08) (width 0.25) (layer "B.Cu") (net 1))
 (segment (start 57.54 25.16) (end 55 25.16) (width 0.25) (layer "B.Cu") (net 1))
 (segment (start 39.2701 25.83) (end 54.33 25.83) (width 0.25) (layer "B.Cu") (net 1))
 (segment (start 28.9575 28.063) (end 37.0371 28.063) (width 0.25) (layer "B.Cu") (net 1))
 (segment (start 72 113) (end 59.625 113) (width 0.25) (layer "B.Cu") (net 1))
 (segment (start 39.2701 25.83) (end 39.2701 24.6554) (width 0.25) (layer "B.Cu") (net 1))
 (segment (start 54.33 25.83) (end 55 25.16) (width 0.25) (layer "B.Cu") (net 1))
 (segment (start 59.625 93) (end 42.625 93) (width 0.25) (layer "B.Cu") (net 1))
 (segment (start 59.625 113) (end 42.625 113) (width 0.25) (layer "B.Cu") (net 1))
 (segment (start 25.625 113) (end 8.625 113) (width 0.25) (layer "B.Cu") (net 1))
 (segment (start 25.625 89.2267) (end 25.0883 89.2267) (width 0.25) (layer "F.Cu") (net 3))
 (segment (start 25.1402 91.75) (end 26.1518 91.75) (width 0.25) (layer "F.Cu") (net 3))
 (segment (start 24.3683 90.9781) (end 25.1402 91.75) (width 0.25) (layer "F.Cu") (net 3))
 (segment (start 24.3683 89.9467) (end 24.3683 90.9781) (width 0.25) (layer "F.Cu") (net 3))
 (segment (start 26.1518 91.75) (end 27.0633 92.6615) (width 0.25) (layer "F.Cu") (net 3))
 (segment (start 25.625 88) (end 25.625 89.2267) (width 0.25) (layer "F.Cu") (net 3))
 (segment (start 27.0633 122.9617) (end 25.625 124.4) (width 0.25) (layer "F.Cu") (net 3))
 (segment (start 27.0633 92.6615) (end 27.0633 122.9617) (width 0.25) (layer "F.Cu") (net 3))
 (segment (start 25.0883 89.2267) (end 24.3683 89.9467) (width 0.25) (layer "F.Cu") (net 3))
 (segment (start 72 116.1) (end 70.443 114.543) (width 0.25) (layer "F.Cu") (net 9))
 (segment (start 72 124.4) (end 72 116.1) (width 0.25) (layer "F.Cu") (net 9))
 (segment (start 70.443 114.543) (end 70.443 58.2621) (width 0.25) (layer "F.Cu") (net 9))
 (via (at 70.443 58.2621) (size 0.6) (drill 0.3) (layers "F.Cu" "B.Cu") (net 9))
 (segment (start 40.2248 52.434) (end 32.514 52.434) (width 0.25) (layer "B.Cu") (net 9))
 (segment (start 40.2248 52.434) (end 46.0529 58.2621) (width 0.25) (layer "B.Cu") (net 9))
 (segment (start 46.0529 58.2621) (end 70.443 58.2621) (width 0.25) (layer "B.Cu") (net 9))
 (segment (start 32.514 52.434) (end 27.62 47.54) (width 0.25) (layer "B.Cu") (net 9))
 (segment (start 27.1698 46.3586) (end 26.4463 47.0821) (width 0.25) (layer "B.Cu") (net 8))
 (segment (start 26.4463 48.9063) (end 27.62 50.08) (width 0.25) (layer "B.Cu") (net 8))
 (segment (start 41.2062 48.4628) (end 39.102 46.3586) (width 0.25) (layer "B.Cu") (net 8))
 (segment (start 30.0648 52.434) (end 27.7108 50.08) (width 0.25) (layer "B.Cu") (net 8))
 (segment (start 39.102 46.3586) (end 27.1698 46.3586) (width 0.25) (layer "B.Cu") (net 8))
 (segment (start 26.4463 47.0821) (end 26.4463 48.9063) (width 0.25) (layer "B.Cu") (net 8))
 (segment (start 27.7108 50.08) (end 27.62 50.08) (width 0.25) (layer "B.Cu") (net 8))
 (segment (start 41.2214 90.0936) (end 41.2214 122.9964) (width 0.25) (layer "F.Cu") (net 15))
 (segment (start 42.625 89.2267) (end 42.0883 89.2267) (width 0.25) (layer "F.Cu") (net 15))
 (segment (start 42.625 88) (end 42.625 89.2267) (width 0.25) (layer "F.Cu") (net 15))
 (segment (start 42.0883 89.2267) (end 41.2214 90.0936) (width 0.25) (layer "F.Cu") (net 15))
 (segment (start 41.2214 122.9964) (end 42.625 124.4) (width 0.25) (layer "F.Cu") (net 15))
 (segment (start 27.4394 65.5) (end 27.4394 88.6856) (width 0.25) (layer "F.Cu") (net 11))
 (segment (start 27.4394 88.6856) (end 25.625 90.5) (width 0.25) (layer "F.Cu") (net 11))
 (segment (start 24.0868 41.4668) (end 27.62 45) (width 0.25) (layer "F.Cu") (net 10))
 (segment (start 24.0868 36.4621) (end 24.0868 41.4668) (width 0.25) (layer "F.Cu") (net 10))
 (segment (start 58.7487 23.8287) (end 58.7487 25.7149) (width 0.25) (layer "B.Cu") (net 10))
 (segment (start 27.2343 33.3146) (end 24.0868 36.4621) (width 0.25) (layer "B.Cu") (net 10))
 (segment (start 58.7487 25.7149) (end 51.149 33.3146) (width 0.25) (layer "B.Cu") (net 10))
 (segment (start 39.5399 33.3146) (end 27.2343 33.3146) (width 0.25) (layer "B.Cu") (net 10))
 (segment (start 57.54 22.62) (end 58.7487 23.8287) (width 0.25) (layer "B.Cu") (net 10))
 (segment (start 51.149 33.3146) (end 39.5399 33.3146) (width 0.25) (layer "B.Cu") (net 10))
 (segment (start 55 22.62) (end 57.54 22.62) (width 0.25) (layer "B.Cu") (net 10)))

